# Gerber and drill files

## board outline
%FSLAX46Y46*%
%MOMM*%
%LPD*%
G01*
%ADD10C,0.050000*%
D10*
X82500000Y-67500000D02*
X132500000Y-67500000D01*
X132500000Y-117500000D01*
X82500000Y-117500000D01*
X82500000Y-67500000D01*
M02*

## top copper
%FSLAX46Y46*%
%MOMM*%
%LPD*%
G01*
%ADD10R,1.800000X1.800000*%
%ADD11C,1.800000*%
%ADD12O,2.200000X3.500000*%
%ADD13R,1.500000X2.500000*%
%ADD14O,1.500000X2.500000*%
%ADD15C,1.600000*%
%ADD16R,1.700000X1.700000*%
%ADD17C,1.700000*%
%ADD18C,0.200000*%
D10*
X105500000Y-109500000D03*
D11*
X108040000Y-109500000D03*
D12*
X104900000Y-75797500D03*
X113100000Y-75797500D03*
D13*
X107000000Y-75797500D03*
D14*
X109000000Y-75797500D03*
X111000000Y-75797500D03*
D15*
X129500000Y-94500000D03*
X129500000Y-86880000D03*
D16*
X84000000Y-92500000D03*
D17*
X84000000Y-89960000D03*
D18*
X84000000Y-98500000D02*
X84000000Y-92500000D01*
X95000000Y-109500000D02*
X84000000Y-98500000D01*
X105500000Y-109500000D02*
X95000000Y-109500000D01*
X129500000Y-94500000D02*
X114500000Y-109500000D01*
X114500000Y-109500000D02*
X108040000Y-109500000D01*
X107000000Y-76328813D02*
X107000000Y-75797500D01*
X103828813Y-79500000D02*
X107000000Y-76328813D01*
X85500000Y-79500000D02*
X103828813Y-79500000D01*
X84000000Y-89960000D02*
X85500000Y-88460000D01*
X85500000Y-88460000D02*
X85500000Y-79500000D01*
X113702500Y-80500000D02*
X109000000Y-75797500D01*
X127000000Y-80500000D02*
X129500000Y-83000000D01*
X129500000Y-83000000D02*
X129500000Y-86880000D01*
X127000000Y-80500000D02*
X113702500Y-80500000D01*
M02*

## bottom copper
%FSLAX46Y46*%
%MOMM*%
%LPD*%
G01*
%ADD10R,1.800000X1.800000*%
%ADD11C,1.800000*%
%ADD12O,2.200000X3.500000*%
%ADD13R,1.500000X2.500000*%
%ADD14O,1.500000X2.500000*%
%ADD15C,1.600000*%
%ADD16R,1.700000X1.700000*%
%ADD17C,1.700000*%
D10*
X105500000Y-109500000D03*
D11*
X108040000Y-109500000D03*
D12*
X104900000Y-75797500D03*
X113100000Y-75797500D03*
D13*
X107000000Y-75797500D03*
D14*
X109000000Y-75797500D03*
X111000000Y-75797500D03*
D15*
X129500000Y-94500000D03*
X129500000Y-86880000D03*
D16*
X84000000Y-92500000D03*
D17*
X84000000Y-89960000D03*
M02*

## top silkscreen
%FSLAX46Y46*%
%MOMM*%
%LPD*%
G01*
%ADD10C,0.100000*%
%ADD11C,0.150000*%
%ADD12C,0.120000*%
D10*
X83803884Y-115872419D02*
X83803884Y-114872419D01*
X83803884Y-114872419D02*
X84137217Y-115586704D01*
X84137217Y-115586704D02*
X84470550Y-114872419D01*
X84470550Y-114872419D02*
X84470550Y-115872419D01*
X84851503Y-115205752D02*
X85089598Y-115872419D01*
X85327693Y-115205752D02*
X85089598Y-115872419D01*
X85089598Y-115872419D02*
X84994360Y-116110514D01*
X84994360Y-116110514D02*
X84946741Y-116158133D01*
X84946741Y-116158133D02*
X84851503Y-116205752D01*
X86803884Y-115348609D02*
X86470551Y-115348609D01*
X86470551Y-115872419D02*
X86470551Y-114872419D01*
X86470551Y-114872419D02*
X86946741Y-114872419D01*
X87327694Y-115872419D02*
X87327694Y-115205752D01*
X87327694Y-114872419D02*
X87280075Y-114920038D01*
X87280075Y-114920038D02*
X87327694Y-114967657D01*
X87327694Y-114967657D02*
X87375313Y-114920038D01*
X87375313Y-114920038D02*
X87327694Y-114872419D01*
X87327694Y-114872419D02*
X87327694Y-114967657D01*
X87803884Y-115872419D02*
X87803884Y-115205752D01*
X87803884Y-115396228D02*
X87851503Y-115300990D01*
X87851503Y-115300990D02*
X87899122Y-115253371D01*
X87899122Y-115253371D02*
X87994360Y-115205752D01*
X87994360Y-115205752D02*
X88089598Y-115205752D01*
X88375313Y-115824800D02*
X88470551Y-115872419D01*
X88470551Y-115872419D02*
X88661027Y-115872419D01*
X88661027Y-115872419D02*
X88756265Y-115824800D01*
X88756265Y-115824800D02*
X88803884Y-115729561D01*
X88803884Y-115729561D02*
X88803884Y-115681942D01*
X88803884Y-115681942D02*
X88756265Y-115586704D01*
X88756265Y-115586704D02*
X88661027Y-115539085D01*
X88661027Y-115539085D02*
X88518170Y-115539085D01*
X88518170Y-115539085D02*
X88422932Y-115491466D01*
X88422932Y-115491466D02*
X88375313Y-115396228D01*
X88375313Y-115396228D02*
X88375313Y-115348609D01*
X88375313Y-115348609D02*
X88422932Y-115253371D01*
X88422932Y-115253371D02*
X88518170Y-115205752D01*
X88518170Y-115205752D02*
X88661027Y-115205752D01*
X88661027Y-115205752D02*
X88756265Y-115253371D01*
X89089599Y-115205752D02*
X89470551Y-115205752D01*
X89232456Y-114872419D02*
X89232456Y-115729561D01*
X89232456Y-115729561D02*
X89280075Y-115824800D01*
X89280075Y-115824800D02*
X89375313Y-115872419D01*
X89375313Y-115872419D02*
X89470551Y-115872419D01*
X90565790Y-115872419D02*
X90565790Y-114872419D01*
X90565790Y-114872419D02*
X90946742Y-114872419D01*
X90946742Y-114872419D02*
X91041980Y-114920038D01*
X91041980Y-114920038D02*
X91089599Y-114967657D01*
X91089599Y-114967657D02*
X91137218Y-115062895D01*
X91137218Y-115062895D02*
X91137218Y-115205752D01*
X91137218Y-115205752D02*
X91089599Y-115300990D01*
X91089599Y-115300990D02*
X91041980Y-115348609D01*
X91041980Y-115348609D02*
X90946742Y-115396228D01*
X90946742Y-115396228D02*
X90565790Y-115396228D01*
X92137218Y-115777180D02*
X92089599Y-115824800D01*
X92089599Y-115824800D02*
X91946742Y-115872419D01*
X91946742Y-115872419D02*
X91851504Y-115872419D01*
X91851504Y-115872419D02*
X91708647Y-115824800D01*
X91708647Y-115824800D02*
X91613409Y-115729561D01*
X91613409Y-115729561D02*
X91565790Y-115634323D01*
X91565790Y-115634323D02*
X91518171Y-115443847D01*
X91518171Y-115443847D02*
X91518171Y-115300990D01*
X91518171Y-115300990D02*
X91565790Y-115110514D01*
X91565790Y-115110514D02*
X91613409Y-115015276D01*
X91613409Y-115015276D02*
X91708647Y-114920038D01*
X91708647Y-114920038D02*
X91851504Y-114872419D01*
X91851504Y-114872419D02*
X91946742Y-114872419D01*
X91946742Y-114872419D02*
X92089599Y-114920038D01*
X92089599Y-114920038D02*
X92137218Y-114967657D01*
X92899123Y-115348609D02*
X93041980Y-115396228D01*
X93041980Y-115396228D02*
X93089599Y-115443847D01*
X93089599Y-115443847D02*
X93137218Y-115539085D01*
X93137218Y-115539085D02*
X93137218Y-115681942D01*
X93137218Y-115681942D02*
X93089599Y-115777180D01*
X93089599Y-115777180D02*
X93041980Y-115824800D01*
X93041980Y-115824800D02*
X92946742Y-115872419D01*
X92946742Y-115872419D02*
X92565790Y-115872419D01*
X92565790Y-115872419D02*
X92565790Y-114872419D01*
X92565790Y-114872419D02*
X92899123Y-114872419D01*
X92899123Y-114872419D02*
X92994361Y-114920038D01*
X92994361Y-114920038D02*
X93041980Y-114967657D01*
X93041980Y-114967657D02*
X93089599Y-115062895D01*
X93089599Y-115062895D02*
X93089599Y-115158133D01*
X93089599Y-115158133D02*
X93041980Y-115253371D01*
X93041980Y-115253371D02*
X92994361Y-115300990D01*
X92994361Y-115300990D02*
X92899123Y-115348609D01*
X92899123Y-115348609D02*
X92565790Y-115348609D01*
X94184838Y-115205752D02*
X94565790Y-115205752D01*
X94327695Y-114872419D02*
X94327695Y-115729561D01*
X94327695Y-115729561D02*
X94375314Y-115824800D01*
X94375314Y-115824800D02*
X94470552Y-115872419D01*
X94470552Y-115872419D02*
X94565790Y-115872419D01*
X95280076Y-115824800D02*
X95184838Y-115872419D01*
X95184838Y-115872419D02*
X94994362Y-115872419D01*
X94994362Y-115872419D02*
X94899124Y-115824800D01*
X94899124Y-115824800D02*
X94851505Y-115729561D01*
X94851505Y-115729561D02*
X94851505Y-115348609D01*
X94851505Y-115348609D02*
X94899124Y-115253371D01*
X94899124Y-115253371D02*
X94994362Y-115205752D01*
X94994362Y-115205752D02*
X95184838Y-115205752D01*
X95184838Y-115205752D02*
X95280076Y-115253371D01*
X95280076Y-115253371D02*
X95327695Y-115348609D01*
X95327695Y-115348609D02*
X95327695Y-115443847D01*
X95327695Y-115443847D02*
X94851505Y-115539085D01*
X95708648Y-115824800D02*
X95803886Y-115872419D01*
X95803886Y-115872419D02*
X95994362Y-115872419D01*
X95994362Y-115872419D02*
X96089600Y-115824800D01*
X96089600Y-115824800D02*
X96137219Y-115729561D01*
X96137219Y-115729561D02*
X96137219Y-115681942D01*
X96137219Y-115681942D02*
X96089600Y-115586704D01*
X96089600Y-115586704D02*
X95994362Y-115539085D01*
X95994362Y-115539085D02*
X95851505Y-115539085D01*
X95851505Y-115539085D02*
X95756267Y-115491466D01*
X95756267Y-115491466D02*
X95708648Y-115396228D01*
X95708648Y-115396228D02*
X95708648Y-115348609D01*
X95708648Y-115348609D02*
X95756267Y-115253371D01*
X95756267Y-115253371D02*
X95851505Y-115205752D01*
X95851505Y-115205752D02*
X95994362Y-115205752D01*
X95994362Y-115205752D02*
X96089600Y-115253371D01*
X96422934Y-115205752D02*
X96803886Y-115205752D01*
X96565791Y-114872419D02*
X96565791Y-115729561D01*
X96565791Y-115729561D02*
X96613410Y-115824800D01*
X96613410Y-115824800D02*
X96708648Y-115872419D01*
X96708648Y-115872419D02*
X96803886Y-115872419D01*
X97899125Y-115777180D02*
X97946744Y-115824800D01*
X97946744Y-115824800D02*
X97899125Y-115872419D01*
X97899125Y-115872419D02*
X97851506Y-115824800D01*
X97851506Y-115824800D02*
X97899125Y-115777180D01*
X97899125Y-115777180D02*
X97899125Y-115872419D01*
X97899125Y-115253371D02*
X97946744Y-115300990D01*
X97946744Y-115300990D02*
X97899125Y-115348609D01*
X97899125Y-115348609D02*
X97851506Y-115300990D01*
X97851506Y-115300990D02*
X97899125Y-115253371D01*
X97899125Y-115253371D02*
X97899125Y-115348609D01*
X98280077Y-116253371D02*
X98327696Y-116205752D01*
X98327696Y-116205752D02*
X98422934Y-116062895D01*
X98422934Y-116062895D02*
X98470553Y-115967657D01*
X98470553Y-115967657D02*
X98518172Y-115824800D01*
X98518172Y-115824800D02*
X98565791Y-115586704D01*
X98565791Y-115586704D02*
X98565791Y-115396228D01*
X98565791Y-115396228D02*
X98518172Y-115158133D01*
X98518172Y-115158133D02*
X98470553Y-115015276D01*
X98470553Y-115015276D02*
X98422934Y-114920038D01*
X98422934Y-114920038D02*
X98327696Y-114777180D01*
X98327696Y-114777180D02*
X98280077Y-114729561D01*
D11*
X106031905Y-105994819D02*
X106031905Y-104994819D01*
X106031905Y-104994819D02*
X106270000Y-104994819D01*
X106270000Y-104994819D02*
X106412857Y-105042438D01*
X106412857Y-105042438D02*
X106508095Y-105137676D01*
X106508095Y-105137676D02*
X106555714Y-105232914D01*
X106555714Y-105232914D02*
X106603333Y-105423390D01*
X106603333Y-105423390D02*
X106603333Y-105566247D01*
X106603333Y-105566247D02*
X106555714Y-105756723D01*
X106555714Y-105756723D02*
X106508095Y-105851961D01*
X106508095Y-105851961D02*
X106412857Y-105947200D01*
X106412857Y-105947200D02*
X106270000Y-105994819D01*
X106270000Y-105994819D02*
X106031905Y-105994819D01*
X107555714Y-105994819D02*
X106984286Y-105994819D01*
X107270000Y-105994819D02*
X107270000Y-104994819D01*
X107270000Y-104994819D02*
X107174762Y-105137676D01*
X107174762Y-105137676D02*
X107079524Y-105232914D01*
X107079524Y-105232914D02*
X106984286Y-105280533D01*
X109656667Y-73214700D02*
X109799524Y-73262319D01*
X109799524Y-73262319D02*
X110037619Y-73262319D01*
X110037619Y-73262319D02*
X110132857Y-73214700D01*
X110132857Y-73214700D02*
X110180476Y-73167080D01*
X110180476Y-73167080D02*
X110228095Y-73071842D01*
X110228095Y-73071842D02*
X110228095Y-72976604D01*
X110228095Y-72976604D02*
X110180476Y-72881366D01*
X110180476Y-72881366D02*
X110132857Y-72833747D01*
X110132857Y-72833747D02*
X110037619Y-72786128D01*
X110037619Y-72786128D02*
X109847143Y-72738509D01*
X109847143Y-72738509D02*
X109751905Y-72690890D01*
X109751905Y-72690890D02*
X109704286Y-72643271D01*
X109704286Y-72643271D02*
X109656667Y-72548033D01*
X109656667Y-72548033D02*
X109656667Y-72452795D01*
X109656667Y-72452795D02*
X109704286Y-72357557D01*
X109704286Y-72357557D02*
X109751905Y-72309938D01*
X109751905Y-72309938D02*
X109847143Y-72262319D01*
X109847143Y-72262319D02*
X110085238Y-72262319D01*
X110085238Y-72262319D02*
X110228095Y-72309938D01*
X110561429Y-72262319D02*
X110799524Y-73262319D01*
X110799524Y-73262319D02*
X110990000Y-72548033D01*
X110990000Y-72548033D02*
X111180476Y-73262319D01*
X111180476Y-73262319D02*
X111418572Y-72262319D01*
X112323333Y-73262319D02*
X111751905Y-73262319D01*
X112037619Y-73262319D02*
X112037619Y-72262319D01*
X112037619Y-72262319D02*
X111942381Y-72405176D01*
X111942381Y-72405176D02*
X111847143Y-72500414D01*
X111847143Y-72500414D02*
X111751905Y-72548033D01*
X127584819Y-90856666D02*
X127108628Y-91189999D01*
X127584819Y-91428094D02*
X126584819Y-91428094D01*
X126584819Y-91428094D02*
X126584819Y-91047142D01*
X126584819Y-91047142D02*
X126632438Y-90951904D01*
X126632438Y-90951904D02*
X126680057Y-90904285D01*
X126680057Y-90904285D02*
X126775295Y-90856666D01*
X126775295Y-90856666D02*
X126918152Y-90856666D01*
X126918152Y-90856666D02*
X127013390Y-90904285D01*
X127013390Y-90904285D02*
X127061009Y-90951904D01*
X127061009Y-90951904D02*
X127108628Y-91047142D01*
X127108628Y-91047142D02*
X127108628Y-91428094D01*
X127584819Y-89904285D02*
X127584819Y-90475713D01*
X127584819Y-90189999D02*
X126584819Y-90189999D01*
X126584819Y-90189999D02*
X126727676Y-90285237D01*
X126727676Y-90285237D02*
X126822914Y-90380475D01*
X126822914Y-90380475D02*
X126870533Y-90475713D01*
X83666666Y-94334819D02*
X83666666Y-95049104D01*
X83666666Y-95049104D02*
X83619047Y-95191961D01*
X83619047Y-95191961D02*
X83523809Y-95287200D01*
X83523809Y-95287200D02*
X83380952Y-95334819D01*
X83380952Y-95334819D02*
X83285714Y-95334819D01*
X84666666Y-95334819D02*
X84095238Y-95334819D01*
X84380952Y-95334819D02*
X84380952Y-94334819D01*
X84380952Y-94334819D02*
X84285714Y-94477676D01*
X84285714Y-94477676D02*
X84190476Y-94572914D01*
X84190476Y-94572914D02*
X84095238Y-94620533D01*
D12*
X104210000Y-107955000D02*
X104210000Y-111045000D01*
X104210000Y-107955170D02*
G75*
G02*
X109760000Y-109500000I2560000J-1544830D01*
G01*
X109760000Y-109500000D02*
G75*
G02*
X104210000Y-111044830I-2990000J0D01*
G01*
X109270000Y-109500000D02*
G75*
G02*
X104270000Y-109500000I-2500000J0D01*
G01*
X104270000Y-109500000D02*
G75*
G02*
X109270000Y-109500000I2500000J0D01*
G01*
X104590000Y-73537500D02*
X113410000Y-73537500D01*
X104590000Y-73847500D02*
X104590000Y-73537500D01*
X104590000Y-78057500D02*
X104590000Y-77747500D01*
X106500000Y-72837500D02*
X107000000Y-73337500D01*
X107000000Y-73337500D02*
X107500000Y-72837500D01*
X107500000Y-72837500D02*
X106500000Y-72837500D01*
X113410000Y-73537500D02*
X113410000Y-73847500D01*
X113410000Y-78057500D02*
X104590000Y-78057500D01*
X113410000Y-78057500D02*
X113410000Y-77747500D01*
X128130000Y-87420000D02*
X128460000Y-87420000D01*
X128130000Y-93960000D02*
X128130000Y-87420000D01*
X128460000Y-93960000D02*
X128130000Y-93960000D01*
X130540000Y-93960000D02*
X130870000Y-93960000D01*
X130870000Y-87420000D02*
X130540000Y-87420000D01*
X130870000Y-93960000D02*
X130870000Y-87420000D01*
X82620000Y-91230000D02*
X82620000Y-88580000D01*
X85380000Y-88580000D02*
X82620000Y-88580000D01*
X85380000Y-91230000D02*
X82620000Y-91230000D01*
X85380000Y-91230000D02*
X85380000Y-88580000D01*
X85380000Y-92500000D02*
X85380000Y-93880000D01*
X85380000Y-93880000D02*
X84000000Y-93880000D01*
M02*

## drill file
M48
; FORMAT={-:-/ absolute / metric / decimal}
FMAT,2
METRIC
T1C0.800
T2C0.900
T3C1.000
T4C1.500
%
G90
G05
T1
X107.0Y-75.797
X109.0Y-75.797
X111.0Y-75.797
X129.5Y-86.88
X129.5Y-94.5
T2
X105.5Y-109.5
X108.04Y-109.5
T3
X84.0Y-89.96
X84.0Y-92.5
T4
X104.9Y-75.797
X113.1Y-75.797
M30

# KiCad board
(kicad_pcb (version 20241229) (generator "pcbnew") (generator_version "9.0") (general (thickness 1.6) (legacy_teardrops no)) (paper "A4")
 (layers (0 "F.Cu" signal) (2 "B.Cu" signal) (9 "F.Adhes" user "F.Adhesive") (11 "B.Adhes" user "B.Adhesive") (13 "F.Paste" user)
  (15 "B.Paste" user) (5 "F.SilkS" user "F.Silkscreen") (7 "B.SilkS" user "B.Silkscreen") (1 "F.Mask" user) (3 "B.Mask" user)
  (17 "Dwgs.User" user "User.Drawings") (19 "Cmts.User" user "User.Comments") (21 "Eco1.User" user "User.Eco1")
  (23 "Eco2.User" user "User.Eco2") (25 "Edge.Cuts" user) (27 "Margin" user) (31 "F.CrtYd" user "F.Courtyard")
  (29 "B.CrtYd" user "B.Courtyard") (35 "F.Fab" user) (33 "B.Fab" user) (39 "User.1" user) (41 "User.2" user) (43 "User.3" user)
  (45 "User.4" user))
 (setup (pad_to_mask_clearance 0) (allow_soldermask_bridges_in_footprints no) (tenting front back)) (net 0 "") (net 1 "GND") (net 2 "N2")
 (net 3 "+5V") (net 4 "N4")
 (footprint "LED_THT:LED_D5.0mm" (layer "F.Cu") (at 105.5 109.5)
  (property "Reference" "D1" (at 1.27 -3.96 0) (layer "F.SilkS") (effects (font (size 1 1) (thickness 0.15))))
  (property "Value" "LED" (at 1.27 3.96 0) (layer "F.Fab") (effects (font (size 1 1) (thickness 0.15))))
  (fp_line (start -1.29 -1.545) (end -1.29 1.545) (stroke (width 0.12) (type solid)) (layer "F.SilkS"))
  (fp_arc (start -1.29 -1.54483) (mid 2.071779 -2.880495) (end 4.26 0) (stroke (width 0.12) (type solid)) (layer "F.SilkS"))
  (fp_arc (start 4.26 0) (mid 2.071779 2.880495) (end -1.29 1.54483) (stroke (width 0.12) (type solid)) (layer "F.SilkS"))
  (fp_circle (center 1.27 0) (end 3.77 0) (stroke (width 0.12) (type solid)) (fill no) (layer "F.SilkS"))
  (pad "1" thru_hole rect (at 0 0) (size 1.8 1.8) (drill 0.9) (layers "*.Cu" "*.Mask") (remove_unused_layers no) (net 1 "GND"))
  (pad "2" thru_hole circle (at 2.54 0) (size 1.8 1.8) (drill 0.9) (layers "*.Cu" "*.Mask") (remove_unused_layers no) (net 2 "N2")))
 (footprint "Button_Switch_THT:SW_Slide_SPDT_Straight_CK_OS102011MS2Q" (layer "F.Cu") (at 107 75.7975)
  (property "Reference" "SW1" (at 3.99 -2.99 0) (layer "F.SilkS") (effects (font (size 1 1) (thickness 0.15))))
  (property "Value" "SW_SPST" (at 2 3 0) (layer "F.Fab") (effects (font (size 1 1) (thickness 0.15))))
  (fp_line (start -2.41 -2.26) (end 6.41 -2.26) (stroke (width 0.12) (type solid)) (layer "F.SilkS"))
  (fp_line (start -2.41 -1.95) (end -2.41 -2.26) (stroke (width 0.12) (type solid)) (layer "F.SilkS"))
  (fp_line (start -2.41 2.26) (end -2.41 1.95) (stroke (width 0.12) (type solid)) (layer "F.SilkS"))
  (fp_line (start -0.5 -2.96) (end 0 -2.46) (stroke (width 0.12) (type solid)) (layer "F.SilkS"))
  (fp_line (start 0 -2.46) (end 0.5 -2.96) (stroke (width 0.12) (type solid)) (layer "F.SilkS"))
  (fp_line (start 0.5 -2.96) (end -0.5 -2.96) (stroke (width 0.12) (type solid)) (layer "F.SilkS"))
  (fp_line (start 6.41 -2.26) (end 6.41 -1.95) (stroke (width 0.12) (type solid)) (layer "F.SilkS"))
  (fp_line (start 6.41 2.26) (end -2.41 2.26) (stroke (width 0.12) (type solid)) (layer "F.SilkS"))
  (fp_line (start 6.41 2.26) (end 6.41 1.95) (stroke (width 0.12) (type solid)) (layer "F.SilkS"))
  (pad "" thru_hole oval (at -2.1 0) (size 2.2 3.5) (drill 1.5) (layers "*.Cu" "*.Mask") (remove_unused_layers no))
  (pad "" thru_hole oval (at 6.1 0) (size 2.2 3.5) (drill 1.5) (layers "*.Cu" "*.Mask") (remove_unused_layers no))
  (pad "1" thru_hole rect (at 0 0) (size 1.5 2.5) (drill 0.8) (layers "*.Cu" "*.Mask") (remove_unused_layers no) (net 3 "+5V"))
  (pad "2" thru_hole oval (at 2 0) (size 1.5 2.5) (drill 0.8) (layers "*.Cu" "*.Mask") (remove_unused_layers no) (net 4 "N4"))
  (pad "3" thru_hole oval (at 4 0) (size 1.5 2.5) (drill 0.8) (layers "*.Cu" "*.Mask") (remove_unused_layers no)))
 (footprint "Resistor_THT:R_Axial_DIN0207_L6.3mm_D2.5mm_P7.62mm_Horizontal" (layer "F.Cu") (at 129.5 94.5 90)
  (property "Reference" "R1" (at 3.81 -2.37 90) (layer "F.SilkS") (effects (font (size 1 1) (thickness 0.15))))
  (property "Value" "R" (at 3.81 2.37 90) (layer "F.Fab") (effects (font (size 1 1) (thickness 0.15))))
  (fp_line (start 7.08 -1.37) (end 7.08 -1.04) (stroke (width 0.12) (type solid)) (layer "F.SilkS"))
  (fp_line (start 0.54 -1.37) (end 7.08 -1.37) (stroke (width 0.12) (type solid)) (layer "F.SilkS"))
  (fp_line (start 0.54 -1.04) (end 0.54 -1.37) (stroke (width 0.12) (type solid)) (layer "F.SilkS"))
  (fp_line (start 0.54 1.04) (end 0.54 1.37) (stroke (width 0.12) (type solid)) (layer "F.SilkS"))
  (fp_line (start 7.08 1.37) (end 7.08 1.04) (stroke (width 0.12) (type solid)) (layer "F.SilkS"))
  (fp_line (start 0.54 1.37) (end 7.08 1.37) (stroke (width 0.12) (type solid)) (layer "F.SilkS"))
  (pad "1" thru_hole circle (at 0 0 90) (size 1.6 1.6) (drill 0.8) (layers "*.Cu" "*.Mask") (remove_unused_layers no) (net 2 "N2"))
  (pad "2" thru_hole circle (at 7.62 0 90) (size 1.6 1.6) (drill 0.8) (layers "*.Cu" "*.Mask") (remove_unused_layers no) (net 4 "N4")))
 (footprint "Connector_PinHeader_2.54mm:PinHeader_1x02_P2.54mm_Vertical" (layer "F.Cu") (at 84 92.5 180)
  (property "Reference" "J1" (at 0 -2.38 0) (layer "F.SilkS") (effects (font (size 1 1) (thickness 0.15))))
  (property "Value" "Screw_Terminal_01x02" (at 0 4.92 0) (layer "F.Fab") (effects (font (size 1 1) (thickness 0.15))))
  (fp_line (start 1.38 1.27) (end 1.38 3.92) (stroke (width 0.12) (type solid)) (layer "F.SilkS"))
  (fp_line (start -1.38 3.92) (end 1.38 3.92) (stroke (width 0.12) (type solid)) (layer "F.SilkS"))
  (fp_line (start -1.38 1.27) (end 1.38 1.27) (stroke (width 0.12) (type solid)) (layer "F.SilkS"))
  (fp_line (start -1.38 1.27) (end -1.38 3.92) (stroke (width 0.12) (type solid)) (layer "F.SilkS"))
  (fp_line (start -1.38 0) (end -1.38 -1.38) (stroke (width 0.12) (type solid)) (layer "F.SilkS"))
  (fp_line (start -1.38 -1.38) (end 0 -1.38) (stroke (width 0.12) (type solid)) (layer "F.SilkS"))
  (pad "1" thru_hole rect (at 0 0 180) (size 1.7 1.7) (drill 1) (layers "*.Cu" "*.Mask") (remove_unused_layers no) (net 1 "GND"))
  (pad "2" thru_hole circle (at 0 2.54 180) (size 1.7 1.7) (drill 1) (layers "*.Cu" "*.Mask") (remove_unused_layers no) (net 3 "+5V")))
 (gr_rect (start 82.5 67.5) (end 132.5 117.5) (stroke (width 0.05) (type solid)) (fill no) (layer "Edge.Cuts"))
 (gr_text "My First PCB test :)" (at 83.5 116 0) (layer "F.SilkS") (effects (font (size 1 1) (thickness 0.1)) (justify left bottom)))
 (segment (start 84 98.5) (end 84 92.5) (width 0.2) (layer "F.Cu") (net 1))
 (segment (start 95 109.5) (end 84 98.5) (width 0.2) (layer "F.Cu") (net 1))
 (segment (start 105.5 109.5) (end 95 109.5) (width 0.2) (layer "F.Cu") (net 1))
 (segment (start 129.5 94.5) (end 114.5 109.5) (width 0.2) (layer "F.Cu") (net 2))
 (segment (start 114.5 109.5) (end 108.04 109.5) (width 0.2) (layer "F.Cu") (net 2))
 (segment (start 107 76.328813) (end 107 75.7975) (width 0.2) (layer "F.Cu") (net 3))
 (segment (start 103.828813 79.5) (end 107 76.328813) (width 0.2) (layer "F.Cu") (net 3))
 (segment (start 85.5 79.5) (end 103.828813 79.5) (width 0.2) (layer "F.Cu") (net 3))
 (segment (start 84 89.96) (end 85.5 88.46) (width 0.2) (layer "F.Cu") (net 3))
 (segment (start 85.5 88.46) (end 85.5 79.5) (width 0.2) (layer "F.Cu") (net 3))
 (segment (start 113.7025 80.5) (end 109 75.7975) (width 0.2) (layer "F.Cu") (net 4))
 (segment (start 127 80.5) (end 129.5 83) (width 0.2) (layer "F.Cu") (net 4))
 (segment (start 129.5 83) (end 129.5 86.88) (width 0.2) (layer "F.Cu") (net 4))
 (segment (start 127 80.5) (end 113.7025 80.5) (width 0.2) (layer "F.Cu") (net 4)))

